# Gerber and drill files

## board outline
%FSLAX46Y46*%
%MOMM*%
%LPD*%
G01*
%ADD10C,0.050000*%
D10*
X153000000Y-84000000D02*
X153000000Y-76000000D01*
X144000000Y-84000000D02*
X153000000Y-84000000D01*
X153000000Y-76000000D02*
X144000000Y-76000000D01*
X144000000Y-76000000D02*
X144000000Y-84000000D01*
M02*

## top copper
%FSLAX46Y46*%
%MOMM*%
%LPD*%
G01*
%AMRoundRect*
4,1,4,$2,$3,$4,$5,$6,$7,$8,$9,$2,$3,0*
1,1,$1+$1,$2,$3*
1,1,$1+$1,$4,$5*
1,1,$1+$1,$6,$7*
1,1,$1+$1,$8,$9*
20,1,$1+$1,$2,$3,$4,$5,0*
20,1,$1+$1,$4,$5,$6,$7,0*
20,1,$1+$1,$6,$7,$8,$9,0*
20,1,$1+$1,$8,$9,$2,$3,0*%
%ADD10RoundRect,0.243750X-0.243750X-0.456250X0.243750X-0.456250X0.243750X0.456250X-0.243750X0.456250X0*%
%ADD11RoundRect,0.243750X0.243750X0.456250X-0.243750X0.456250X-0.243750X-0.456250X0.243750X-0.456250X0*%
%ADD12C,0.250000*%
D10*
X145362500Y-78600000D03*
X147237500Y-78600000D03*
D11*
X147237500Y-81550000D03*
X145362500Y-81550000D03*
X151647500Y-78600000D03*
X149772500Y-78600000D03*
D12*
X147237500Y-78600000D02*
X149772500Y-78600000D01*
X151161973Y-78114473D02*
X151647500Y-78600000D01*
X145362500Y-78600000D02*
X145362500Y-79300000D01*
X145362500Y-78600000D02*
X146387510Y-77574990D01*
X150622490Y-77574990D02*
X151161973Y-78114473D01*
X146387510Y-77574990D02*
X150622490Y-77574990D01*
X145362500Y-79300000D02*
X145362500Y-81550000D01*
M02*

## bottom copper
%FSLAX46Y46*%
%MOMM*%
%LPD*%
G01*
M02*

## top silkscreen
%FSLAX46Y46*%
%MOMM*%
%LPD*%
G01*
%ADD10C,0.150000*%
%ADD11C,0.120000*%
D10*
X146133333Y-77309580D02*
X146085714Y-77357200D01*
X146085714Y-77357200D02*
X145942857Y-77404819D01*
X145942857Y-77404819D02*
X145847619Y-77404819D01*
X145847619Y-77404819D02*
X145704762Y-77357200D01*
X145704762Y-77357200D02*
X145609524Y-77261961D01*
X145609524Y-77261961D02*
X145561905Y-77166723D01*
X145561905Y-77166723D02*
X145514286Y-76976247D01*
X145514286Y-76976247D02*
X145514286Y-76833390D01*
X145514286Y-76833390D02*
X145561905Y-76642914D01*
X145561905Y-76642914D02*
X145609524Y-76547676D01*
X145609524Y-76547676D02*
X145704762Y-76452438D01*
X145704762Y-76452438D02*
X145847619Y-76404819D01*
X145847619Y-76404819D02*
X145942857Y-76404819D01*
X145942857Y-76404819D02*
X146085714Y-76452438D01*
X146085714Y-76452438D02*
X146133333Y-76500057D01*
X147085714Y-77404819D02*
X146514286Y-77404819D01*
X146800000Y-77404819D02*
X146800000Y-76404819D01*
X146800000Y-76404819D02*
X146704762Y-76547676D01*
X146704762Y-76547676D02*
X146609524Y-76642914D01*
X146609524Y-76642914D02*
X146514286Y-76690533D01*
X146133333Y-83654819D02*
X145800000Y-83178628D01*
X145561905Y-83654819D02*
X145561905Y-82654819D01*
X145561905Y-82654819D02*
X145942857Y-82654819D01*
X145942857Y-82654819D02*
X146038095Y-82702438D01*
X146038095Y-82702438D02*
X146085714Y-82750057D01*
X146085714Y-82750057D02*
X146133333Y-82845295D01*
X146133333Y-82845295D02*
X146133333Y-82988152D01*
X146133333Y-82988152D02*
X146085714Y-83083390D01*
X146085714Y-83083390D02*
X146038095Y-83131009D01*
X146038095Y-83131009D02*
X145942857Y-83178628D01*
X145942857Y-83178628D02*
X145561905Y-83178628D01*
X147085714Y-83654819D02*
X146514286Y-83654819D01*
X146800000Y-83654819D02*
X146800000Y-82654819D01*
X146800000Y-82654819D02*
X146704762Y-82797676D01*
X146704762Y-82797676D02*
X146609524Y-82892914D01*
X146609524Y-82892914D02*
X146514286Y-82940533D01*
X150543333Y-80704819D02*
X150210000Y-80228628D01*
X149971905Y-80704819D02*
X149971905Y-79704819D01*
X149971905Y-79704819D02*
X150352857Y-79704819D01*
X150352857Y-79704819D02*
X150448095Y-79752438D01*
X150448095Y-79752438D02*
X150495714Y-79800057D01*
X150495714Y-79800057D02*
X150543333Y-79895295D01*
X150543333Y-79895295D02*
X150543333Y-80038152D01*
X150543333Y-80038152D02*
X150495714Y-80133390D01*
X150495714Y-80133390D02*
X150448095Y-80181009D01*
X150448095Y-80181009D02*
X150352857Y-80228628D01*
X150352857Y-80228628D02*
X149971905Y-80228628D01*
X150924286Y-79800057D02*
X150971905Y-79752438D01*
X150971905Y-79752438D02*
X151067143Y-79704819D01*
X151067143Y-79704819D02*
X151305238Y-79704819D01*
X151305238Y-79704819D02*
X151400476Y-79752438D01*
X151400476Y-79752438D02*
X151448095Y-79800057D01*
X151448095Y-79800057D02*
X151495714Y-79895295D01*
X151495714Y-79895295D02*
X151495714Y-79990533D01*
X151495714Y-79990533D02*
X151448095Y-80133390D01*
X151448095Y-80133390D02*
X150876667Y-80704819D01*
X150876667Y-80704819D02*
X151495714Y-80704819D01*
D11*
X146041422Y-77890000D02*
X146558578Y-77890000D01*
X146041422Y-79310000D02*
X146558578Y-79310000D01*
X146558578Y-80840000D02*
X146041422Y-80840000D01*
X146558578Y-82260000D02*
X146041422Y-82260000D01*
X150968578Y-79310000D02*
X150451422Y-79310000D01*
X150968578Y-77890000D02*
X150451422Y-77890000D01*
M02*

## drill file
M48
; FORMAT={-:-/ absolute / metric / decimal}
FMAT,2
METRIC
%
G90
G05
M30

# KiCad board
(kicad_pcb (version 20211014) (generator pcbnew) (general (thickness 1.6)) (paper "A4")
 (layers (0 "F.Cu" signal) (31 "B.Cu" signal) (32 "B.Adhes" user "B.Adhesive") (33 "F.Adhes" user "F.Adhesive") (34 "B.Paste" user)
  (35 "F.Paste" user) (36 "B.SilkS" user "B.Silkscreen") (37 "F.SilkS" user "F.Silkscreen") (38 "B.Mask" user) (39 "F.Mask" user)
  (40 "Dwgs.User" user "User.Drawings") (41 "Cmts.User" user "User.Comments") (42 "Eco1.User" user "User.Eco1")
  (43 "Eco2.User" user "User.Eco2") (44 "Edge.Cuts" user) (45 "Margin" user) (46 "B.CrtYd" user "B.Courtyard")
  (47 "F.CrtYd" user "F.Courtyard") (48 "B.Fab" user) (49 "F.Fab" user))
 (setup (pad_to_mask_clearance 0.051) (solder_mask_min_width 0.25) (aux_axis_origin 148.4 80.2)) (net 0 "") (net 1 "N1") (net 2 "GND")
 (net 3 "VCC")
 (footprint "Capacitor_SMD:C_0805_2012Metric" (layer "F.Cu") (at 146.3 78.6)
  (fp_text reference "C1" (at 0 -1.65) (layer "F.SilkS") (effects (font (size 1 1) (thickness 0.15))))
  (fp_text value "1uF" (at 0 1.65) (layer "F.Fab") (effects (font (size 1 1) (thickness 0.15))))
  (fp_line (start -0.258578 -0.71) (end 0.258578 -0.71) (layer "F.SilkS") (width 0.12))
  (fp_line (start -0.258578 0.71) (end 0.258578 0.71) (layer "F.SilkS") (width 0.12))
  (pad "1" smd roundrect locked (at -0.9375 0) (size 0.975 1.4) (layers "F.Cu" "F.Paste" "F.Mask") (roundrect_rratio 0.25) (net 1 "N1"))
  (pad "2" smd roundrect locked (at 0.9375 0) (size 0.975 1.4) (layers "F.Cu" "F.Paste" "F.Mask") (roundrect_rratio 0.25) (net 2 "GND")))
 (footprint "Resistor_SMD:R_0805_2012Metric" (layer "F.Cu") (at 146.3 81.55 180)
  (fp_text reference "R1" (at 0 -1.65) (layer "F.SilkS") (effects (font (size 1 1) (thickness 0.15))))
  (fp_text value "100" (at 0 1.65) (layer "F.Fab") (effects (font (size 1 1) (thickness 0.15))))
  (fp_line (start -0.258578 0.71) (end 0.258578 0.71) (layer "F.SilkS") (width 0.12))
  (fp_line (start -0.258578 -0.71) (end 0.258578 -0.71) (layer "F.SilkS") (width 0.12))
  (pad "1" smd roundrect locked (at -0.9375 0 180) (size 0.975 1.4) (layers "F.Cu" "F.Paste" "F.Mask") (roundrect_rratio 0.25) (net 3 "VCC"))
  (pad "2" smd roundrect locked (at 0.9375 0 180) (size 0.975 1.4) (layers "F.Cu" "F.Paste" "F.Mask") (roundrect_rratio 0.25) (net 1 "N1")))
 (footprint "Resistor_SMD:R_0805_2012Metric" (layer "F.Cu") (at 150.71 78.6 180)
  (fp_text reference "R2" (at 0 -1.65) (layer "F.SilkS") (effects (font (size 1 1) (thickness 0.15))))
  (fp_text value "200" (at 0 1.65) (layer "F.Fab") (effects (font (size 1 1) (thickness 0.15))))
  (fp_line (start -0.258578 -0.71) (end 0.258578 -0.71) (layer "F.SilkS") (width 0.12))
  (fp_line (start -0.258578 0.71) (end 0.258578 0.71) (layer "F.SilkS") (width 0.12))
  (pad "1" smd roundrect locked (at -0.9375 0 180) (size 0.975 1.4) (layers "F.Cu" "F.Paste" "F.Mask") (roundrect_rratio 0.25) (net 1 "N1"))
  (pad "2" smd roundrect locked (at 0.9375 0 180) (size 0.975 1.4) (layers "F.Cu" "F.Paste" "F.Mask") (roundrect_rratio 0.25) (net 2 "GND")))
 (gr_line (start 153 84) (end 153 76) (layer "Edge.Cuts") (width 0.05))
 (gr_line (start 144 84) (end 153 84) (layer "Edge.Cuts") (width 0.05))
 (gr_line (start 153 76) (end 144 76) (layer "Edge.Cuts") (width 0.05))
 (gr_line (start 144 76) (end 144 84) (layer "Edge.Cuts") (width 0.05))
 (segment (start 147.2375 78.6) (end 149.7725 78.6) (width 0.25) (layer "F.Cu") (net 2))
 (segment (start 151.161973 78.114473) (end 151.6475 78.6) (width 0.25) (layer "F.Cu") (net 1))
 (segment (start 145.3625 78.6) (end 145.3625 79.3) (width 0.25) (layer "F.Cu") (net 1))
 (segment (start 145.3625 78.6) (end 146.38751 77.57499) (width 0.25) (layer "F.Cu") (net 1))
 (segment (start 150.62249 77.57499) (end 151.161973 78.114473) (width 0.25) (layer "F.Cu") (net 1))
 (segment (start 146.38751 77.57499) (end 150.62249 77.57499) (width 0.25) (layer "F.Cu") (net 1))
 (segment (start 145.3625 79.3) (end 145.3625 81.55) (width 0.25) (layer "F.Cu") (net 1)))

